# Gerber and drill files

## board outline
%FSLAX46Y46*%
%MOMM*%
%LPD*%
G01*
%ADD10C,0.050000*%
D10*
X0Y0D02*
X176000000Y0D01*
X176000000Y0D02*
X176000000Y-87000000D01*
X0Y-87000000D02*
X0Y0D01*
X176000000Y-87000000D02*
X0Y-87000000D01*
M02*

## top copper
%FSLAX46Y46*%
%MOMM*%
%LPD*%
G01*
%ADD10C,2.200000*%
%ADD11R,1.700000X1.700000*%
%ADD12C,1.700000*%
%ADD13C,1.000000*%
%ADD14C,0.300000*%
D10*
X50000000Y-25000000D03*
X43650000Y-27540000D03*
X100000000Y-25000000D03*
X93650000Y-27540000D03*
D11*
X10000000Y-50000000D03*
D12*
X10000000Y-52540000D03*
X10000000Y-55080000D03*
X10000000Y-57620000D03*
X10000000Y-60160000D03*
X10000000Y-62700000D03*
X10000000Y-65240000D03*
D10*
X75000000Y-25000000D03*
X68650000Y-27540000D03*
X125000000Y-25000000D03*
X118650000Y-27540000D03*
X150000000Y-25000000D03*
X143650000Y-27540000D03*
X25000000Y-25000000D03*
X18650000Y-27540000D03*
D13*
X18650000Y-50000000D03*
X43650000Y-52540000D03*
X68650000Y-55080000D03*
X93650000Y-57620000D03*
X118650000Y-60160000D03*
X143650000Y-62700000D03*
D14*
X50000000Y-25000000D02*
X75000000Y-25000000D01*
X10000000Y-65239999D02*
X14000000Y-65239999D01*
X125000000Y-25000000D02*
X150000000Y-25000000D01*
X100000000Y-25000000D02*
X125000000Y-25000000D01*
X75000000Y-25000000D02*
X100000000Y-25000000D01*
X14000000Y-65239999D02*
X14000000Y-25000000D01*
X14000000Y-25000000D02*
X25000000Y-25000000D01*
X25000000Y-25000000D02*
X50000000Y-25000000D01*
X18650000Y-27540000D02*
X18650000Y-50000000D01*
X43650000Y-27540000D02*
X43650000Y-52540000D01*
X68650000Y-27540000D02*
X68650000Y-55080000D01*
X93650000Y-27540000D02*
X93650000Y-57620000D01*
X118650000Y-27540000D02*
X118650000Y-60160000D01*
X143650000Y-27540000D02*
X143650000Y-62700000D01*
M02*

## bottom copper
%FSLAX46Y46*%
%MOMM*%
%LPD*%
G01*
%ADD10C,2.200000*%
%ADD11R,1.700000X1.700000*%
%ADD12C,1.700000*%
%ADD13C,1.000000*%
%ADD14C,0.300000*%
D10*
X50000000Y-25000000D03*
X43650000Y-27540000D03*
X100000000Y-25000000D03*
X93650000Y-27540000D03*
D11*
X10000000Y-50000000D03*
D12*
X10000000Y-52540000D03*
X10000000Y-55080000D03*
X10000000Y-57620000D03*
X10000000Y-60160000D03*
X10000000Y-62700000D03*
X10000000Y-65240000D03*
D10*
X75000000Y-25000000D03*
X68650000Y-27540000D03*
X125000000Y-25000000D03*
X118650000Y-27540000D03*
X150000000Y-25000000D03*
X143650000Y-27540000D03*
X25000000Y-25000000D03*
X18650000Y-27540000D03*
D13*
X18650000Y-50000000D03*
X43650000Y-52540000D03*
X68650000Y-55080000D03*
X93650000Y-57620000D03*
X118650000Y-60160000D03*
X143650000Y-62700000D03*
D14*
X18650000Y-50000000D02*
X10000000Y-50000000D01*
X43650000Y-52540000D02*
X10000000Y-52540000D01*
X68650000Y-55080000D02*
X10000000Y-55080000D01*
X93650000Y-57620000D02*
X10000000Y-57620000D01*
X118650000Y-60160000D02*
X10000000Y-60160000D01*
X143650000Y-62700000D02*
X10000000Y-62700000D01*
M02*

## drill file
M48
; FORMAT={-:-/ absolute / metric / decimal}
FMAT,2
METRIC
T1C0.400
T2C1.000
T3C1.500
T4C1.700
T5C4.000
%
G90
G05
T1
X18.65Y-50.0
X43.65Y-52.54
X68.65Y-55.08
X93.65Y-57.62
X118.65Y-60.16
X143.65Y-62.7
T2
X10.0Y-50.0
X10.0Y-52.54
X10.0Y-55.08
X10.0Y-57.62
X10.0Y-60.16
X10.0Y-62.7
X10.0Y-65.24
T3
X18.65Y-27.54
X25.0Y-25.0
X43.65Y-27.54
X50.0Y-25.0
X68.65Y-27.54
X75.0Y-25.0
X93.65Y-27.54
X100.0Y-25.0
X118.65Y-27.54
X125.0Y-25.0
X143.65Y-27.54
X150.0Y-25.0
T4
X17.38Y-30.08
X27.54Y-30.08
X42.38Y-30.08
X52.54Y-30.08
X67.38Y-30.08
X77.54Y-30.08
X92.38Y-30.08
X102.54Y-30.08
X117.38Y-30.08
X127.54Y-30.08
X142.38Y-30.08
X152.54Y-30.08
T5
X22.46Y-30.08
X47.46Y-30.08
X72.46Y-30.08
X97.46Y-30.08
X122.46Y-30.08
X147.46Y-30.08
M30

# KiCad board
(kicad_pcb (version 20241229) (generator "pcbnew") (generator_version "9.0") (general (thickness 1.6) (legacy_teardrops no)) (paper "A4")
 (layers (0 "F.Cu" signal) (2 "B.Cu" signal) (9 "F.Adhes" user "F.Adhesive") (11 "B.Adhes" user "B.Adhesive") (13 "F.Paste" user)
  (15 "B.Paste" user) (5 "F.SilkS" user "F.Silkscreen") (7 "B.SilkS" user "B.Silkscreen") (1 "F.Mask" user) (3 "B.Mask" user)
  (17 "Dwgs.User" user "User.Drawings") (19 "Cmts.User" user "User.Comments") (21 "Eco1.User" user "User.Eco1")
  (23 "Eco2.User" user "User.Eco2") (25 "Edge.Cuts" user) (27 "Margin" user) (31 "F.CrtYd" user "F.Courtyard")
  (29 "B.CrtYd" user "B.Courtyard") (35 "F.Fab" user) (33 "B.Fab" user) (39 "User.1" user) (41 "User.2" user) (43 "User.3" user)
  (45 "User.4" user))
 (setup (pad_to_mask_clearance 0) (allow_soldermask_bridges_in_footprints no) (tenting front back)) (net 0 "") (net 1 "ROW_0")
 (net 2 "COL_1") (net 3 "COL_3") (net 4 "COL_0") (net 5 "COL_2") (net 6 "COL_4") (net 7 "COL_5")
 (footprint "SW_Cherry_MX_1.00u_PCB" (layer "F.Cu") (at 50 25)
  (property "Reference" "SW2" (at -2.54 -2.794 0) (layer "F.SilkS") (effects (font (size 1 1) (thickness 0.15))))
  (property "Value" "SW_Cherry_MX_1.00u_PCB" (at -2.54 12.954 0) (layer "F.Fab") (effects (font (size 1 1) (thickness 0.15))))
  (pad "" np_thru_hole circle (at -7.62 5.08) (size 1.7 1.7) (drill 1.7) (layers "*.Cu" "*.Mask"))
  (pad "" np_thru_hole circle (at -2.54 5.08) (size 4 4) (drill 4) (layers "*.Cu" "*.Mask"))
  (pad "" np_thru_hole circle (at 2.54 5.08) (size 1.7 1.7) (drill 1.7) (layers "*.Cu" "*.Mask"))
  (pad "1" thru_hole circle (at 0 0) (size 2.2 2.2) (drill 1.5) (layers "*.Cu" "*.Mask") (remove_unused_layers no) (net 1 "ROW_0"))
  (pad "2" thru_hole circle (at -6.35 2.54) (size 2.2 2.2) (drill 1.5) (layers "*.Cu" "*.Mask") (remove_unused_layers no) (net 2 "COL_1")))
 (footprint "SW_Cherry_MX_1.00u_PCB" (layer "F.Cu") (at 100 25)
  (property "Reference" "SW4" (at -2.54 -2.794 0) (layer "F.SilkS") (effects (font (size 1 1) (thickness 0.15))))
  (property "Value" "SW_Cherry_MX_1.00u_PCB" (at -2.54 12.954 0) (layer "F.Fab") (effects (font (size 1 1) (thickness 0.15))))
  (pad "" np_thru_hole circle (at -7.62 5.08) (size 1.7 1.7) (drill 1.7) (layers "*.Cu" "*.Mask"))
  (pad "" np_thru_hole circle (at -2.54 5.08) (size 4 4) (drill 4) (layers "*.Cu" "*.Mask"))
  (pad "" np_thru_hole circle (at 2.54 5.08) (size 1.7 1.7) (drill 1.7) (layers "*.Cu" "*.Mask"))
  (pad "1" thru_hole circle (at 0 0) (size 2.2 2.2) (drill 1.5) (layers "*.Cu" "*.Mask") (remove_unused_layers no) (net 1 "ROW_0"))
  (pad "2" thru_hole circle (at -6.35 2.54) (size 2.2 2.2) (drill 1.5) (layers "*.Cu" "*.Mask") (remove_unused_layers no) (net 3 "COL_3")))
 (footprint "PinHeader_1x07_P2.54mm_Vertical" (layer "F.Cu") (at 10 50)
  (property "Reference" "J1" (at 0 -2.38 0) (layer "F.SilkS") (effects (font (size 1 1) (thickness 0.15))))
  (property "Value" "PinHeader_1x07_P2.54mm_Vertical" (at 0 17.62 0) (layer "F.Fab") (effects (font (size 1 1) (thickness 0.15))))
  (pad "1" thru_hole rect (at 0 0) (size 1.7 1.7) (drill 1) (layers "*.Cu" "*.Mask") (remove_unused_layers no) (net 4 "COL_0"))
  (pad "2" thru_hole circle (at 0 2.54) (size 1.7 1.7) (drill 1) (layers "*.Cu" "*.Mask") (remove_unused_layers no) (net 2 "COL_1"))
  (pad "3" thru_hole circle (at 0 5.08) (size 1.7 1.7) (drill 1) (layers "*.Cu" "*.Mask") (remove_unused_layers no) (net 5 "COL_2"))
  (pad "4" thru_hole circle (at 0 7.62) (size 1.7 1.7) (drill 1) (layers "*.Cu" "*.Mask") (remove_unused_layers no) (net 3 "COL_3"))
  (pad "5" thru_hole circle (at 0 10.16) (size 1.7 1.7) (drill 1) (layers "*.Cu" "*.Mask") (remove_unused_layers no) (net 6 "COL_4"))
  (pad "6" thru_hole circle (at 0 12.7) (size 1.7 1.7) (drill 1) (layers "*.Cu" "*.Mask") (remove_unused_layers no) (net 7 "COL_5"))
  (pad "7" thru_hole circle (at 0 15.24) (size 1.7 1.7) (drill 1) (layers "*.Cu" "*.Mask") (remove_unused_layers no) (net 1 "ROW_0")))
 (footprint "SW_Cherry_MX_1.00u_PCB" (layer "F.Cu") (at 75 25)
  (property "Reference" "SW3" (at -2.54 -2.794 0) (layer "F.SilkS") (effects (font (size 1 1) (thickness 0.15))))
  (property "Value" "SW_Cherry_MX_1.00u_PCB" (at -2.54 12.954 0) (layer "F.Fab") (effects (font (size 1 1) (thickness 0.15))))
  (pad "" np_thru_hole circle (at -7.62 5.08) (size 1.7 1.7) (drill 1.7) (layers "*.Cu" "*.Mask"))
  (pad "" np_thru_hole circle (at -2.54 5.08) (size 4 4) (drill 4) (layers "*.Cu" "*.Mask"))
  (pad "" np_thru_hole circle (at 2.54 5.08) (size 1.7 1.7) (drill 1.7) (layers "*.Cu" "*.Mask"))
  (pad "1" thru_hole circle (at 0 0) (size 2.2 2.2) (drill 1.5) (layers "*.Cu" "*.Mask") (remove_unused_layers no) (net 1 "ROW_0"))
  (pad "2" thru_hole circle (at -6.35 2.54) (size 2.2 2.2) (drill 1.5) (layers "*.Cu" "*.Mask") (remove_unused_layers no) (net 5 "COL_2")))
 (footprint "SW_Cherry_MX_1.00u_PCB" (layer "F.Cu") (at 125 25)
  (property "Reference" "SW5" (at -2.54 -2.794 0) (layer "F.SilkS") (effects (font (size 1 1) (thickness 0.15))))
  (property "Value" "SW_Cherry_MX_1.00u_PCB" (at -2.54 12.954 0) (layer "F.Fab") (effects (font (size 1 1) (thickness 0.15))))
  (pad "" np_thru_hole circle (at -7.62 5.08) (size 1.7 1.7) (drill 1.7) (layers "*.Cu" "*.Mask"))
  (pad "" np_thru_hole circle (at -2.54 5.08) (size 4 4) (drill 4) (layers "*.Cu" "*.Mask"))
  (pad "" np_thru_hole circle (at 2.54 5.08) (size 1.7 1.7) (drill 1.7) (layers "*.Cu" "*.Mask"))
  (pad "1" thru_hole circle (at 0 0) (size 2.2 2.2) (drill 1.5) (layers "*.Cu" "*.Mask") (remove_unused_layers no) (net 1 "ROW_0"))
  (pad "2" thru_hole circle (at -6.35 2.54) (size 2.2 2.2) (drill 1.5) (layers "*.Cu" "*.Mask") (remove_unused_layers no) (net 6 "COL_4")))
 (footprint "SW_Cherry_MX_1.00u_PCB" (layer "F.Cu") (at 150 25)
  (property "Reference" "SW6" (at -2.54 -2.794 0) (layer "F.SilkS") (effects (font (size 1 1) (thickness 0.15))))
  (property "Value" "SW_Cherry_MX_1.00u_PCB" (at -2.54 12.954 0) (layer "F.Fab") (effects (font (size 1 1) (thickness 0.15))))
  (pad "" np_thru_hole circle (at -7.62 5.08) (size 1.7 1.7) (drill 1.7) (layers "*.Cu" "*.Mask"))
  (pad "" np_thru_hole circle (at -2.54 5.08) (size 4 4) (drill 4) (layers "*.Cu" "*.Mask"))
  (pad "" np_thru_hole circle (at 2.54 5.08) (size 1.7 1.7) (drill 1.7) (layers "*.Cu" "*.Mask"))
  (pad "1" thru_hole circle (at 0 0) (size 2.2 2.2) (drill 1.5) (layers "*.Cu" "*.Mask") (remove_unused_layers no) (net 1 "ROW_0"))
  (pad "2" thru_hole circle (at -6.35 2.54) (size 2.2 2.2) (drill 1.5) (layers "*.Cu" "*.Mask") (remove_unused_layers no) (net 7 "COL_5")))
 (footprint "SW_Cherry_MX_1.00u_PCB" (layer "F.Cu") (at 25 25)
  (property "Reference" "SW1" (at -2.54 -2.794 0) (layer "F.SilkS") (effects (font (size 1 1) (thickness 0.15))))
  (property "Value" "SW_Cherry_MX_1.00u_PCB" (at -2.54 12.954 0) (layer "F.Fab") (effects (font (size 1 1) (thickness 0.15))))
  (pad "" np_thru_hole circle (at -7.62 5.08) (size 1.7 1.7) (drill 1.7) (layers "*.Cu" "*.Mask"))
  (pad "" np_thru_hole circle (at -2.54 5.08) (size 4 4) (drill 4) (layers "*.Cu" "*.Mask"))
  (pad "" np_thru_hole circle (at 2.54 5.08) (size 1.7 1.7) (drill 1.7) (layers "*.Cu" "*.Mask"))
  (pad "1" thru_hole circle (at 0 0) (size 2.2 2.2) (drill 1.5) (layers "*.Cu" "*.Mask") (remove_unused_layers no) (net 1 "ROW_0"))
  (pad "2" thru_hole circle (at -6.35 2.54) (size 2.2 2.2) (drill 1.5) (layers "*.Cu" "*.Mask") (remove_unused_layers no) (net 4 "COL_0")))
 (gr_line (start 0 0) (end 176 0) (stroke (width 0.05) (type default)) (layer "Edge.Cuts"))
 (gr_line (start 176 0) (end 176 87) (stroke (width 0.05) (type default)) (layer "Edge.Cuts"))
 (gr_line (start 0 87) (end 0 0) (stroke (width 0.05) (type default)) (layer "Edge.Cuts"))
 (gr_line (start 176 87) (end 0 87) (stroke (width 0.05) (type default)) (layer "Edge.Cuts"))
 (segment (start 50 25) (end 75 25) (width 0.3) (layer "F.Cu") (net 1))
 (segment (start 10 65.239999) (end 14 65.239999) (width 0.3) (layer "F.Cu") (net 1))
 (segment (start 125 25) (end 150 25) (width 0.3) (layer "F.Cu") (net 1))
 (segment (start 100 25) (end 125 25) (width 0.3) (layer "F.Cu") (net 1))
 (segment (start 75 25) (end 100 25) (width 0.3) (layer "F.Cu") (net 1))
 (segment (start 14 65.239999) (end 14 25) (width 0.3) (layer "F.Cu") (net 1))
 (segment (start 14 25) (end 25 25) (width 0.3) (layer "F.Cu") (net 1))
 (segment (start 25 25) (end 50 25) (width 0.3) (layer "F.Cu") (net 1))
 (segment (start 18.65 27.54) (end 18.65 50) (width 0.3) (layer "F.Cu") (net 4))
 (via (at 18.65 50) (size 1) (drill 0.4) (layers "F.Cu" "B.Cu") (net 4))
 (segment (start 18.65 50) (end 10 50) (width 0.3) (layer "B.Cu") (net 4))
 (segment (start 43.65 27.54) (end 43.65 52.54) (width 0.3) (layer "F.Cu") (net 2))
 (via (at 43.65 52.54) (size 1) (drill 0.4) (layers "F.Cu" "B.Cu") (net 2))
 (segment (start 43.65 52.54) (end 10 52.54) (width 0.3) (layer "B.Cu") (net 2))
 (segment (start 68.65 27.54) (end 68.65 55.08) (width 0.3) (layer "F.Cu") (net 5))
 (via (at 68.65 55.08) (size 1) (drill 0.4) (layers "F.Cu" "B.Cu") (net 5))
 (segment (start 68.65 55.08) (end 10 55.08) (width 0.3) (layer "B.Cu") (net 5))
 (segment (start 93.65 27.54) (end 93.65 57.62) (width 0.3) (layer "F.Cu") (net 3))
 (via (at 93.65 57.62) (size 1) (drill 0.4) (layers "F.Cu" "B.Cu") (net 3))
 (segment (start 93.65 57.62) (end 10 57.62) (width 0.3) (layer "B.Cu") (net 3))
 (segment (start 118.65 27.54) (end 118.65 60.16) (width 0.3) (layer "F.Cu") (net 6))
 (via (at 118.65 60.16) (size 1) (drill 0.4) (layers "F.Cu" "B.Cu") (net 6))
 (segment (start 118.65 60.16) (end 10 60.16) (width 0.3) (layer "B.Cu") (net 6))
 (segment (start 143.65 27.54) (end 143.65 62.7) (width 0.3) (layer "F.Cu") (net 7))
 (via (at 143.65 62.7) (size 1) (drill 0.4) (layers "F.Cu" "B.Cu") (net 7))
 (segment (start 143.65 62.7) (end 10 62.7) (width 0.3) (layer "B.Cu") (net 7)))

